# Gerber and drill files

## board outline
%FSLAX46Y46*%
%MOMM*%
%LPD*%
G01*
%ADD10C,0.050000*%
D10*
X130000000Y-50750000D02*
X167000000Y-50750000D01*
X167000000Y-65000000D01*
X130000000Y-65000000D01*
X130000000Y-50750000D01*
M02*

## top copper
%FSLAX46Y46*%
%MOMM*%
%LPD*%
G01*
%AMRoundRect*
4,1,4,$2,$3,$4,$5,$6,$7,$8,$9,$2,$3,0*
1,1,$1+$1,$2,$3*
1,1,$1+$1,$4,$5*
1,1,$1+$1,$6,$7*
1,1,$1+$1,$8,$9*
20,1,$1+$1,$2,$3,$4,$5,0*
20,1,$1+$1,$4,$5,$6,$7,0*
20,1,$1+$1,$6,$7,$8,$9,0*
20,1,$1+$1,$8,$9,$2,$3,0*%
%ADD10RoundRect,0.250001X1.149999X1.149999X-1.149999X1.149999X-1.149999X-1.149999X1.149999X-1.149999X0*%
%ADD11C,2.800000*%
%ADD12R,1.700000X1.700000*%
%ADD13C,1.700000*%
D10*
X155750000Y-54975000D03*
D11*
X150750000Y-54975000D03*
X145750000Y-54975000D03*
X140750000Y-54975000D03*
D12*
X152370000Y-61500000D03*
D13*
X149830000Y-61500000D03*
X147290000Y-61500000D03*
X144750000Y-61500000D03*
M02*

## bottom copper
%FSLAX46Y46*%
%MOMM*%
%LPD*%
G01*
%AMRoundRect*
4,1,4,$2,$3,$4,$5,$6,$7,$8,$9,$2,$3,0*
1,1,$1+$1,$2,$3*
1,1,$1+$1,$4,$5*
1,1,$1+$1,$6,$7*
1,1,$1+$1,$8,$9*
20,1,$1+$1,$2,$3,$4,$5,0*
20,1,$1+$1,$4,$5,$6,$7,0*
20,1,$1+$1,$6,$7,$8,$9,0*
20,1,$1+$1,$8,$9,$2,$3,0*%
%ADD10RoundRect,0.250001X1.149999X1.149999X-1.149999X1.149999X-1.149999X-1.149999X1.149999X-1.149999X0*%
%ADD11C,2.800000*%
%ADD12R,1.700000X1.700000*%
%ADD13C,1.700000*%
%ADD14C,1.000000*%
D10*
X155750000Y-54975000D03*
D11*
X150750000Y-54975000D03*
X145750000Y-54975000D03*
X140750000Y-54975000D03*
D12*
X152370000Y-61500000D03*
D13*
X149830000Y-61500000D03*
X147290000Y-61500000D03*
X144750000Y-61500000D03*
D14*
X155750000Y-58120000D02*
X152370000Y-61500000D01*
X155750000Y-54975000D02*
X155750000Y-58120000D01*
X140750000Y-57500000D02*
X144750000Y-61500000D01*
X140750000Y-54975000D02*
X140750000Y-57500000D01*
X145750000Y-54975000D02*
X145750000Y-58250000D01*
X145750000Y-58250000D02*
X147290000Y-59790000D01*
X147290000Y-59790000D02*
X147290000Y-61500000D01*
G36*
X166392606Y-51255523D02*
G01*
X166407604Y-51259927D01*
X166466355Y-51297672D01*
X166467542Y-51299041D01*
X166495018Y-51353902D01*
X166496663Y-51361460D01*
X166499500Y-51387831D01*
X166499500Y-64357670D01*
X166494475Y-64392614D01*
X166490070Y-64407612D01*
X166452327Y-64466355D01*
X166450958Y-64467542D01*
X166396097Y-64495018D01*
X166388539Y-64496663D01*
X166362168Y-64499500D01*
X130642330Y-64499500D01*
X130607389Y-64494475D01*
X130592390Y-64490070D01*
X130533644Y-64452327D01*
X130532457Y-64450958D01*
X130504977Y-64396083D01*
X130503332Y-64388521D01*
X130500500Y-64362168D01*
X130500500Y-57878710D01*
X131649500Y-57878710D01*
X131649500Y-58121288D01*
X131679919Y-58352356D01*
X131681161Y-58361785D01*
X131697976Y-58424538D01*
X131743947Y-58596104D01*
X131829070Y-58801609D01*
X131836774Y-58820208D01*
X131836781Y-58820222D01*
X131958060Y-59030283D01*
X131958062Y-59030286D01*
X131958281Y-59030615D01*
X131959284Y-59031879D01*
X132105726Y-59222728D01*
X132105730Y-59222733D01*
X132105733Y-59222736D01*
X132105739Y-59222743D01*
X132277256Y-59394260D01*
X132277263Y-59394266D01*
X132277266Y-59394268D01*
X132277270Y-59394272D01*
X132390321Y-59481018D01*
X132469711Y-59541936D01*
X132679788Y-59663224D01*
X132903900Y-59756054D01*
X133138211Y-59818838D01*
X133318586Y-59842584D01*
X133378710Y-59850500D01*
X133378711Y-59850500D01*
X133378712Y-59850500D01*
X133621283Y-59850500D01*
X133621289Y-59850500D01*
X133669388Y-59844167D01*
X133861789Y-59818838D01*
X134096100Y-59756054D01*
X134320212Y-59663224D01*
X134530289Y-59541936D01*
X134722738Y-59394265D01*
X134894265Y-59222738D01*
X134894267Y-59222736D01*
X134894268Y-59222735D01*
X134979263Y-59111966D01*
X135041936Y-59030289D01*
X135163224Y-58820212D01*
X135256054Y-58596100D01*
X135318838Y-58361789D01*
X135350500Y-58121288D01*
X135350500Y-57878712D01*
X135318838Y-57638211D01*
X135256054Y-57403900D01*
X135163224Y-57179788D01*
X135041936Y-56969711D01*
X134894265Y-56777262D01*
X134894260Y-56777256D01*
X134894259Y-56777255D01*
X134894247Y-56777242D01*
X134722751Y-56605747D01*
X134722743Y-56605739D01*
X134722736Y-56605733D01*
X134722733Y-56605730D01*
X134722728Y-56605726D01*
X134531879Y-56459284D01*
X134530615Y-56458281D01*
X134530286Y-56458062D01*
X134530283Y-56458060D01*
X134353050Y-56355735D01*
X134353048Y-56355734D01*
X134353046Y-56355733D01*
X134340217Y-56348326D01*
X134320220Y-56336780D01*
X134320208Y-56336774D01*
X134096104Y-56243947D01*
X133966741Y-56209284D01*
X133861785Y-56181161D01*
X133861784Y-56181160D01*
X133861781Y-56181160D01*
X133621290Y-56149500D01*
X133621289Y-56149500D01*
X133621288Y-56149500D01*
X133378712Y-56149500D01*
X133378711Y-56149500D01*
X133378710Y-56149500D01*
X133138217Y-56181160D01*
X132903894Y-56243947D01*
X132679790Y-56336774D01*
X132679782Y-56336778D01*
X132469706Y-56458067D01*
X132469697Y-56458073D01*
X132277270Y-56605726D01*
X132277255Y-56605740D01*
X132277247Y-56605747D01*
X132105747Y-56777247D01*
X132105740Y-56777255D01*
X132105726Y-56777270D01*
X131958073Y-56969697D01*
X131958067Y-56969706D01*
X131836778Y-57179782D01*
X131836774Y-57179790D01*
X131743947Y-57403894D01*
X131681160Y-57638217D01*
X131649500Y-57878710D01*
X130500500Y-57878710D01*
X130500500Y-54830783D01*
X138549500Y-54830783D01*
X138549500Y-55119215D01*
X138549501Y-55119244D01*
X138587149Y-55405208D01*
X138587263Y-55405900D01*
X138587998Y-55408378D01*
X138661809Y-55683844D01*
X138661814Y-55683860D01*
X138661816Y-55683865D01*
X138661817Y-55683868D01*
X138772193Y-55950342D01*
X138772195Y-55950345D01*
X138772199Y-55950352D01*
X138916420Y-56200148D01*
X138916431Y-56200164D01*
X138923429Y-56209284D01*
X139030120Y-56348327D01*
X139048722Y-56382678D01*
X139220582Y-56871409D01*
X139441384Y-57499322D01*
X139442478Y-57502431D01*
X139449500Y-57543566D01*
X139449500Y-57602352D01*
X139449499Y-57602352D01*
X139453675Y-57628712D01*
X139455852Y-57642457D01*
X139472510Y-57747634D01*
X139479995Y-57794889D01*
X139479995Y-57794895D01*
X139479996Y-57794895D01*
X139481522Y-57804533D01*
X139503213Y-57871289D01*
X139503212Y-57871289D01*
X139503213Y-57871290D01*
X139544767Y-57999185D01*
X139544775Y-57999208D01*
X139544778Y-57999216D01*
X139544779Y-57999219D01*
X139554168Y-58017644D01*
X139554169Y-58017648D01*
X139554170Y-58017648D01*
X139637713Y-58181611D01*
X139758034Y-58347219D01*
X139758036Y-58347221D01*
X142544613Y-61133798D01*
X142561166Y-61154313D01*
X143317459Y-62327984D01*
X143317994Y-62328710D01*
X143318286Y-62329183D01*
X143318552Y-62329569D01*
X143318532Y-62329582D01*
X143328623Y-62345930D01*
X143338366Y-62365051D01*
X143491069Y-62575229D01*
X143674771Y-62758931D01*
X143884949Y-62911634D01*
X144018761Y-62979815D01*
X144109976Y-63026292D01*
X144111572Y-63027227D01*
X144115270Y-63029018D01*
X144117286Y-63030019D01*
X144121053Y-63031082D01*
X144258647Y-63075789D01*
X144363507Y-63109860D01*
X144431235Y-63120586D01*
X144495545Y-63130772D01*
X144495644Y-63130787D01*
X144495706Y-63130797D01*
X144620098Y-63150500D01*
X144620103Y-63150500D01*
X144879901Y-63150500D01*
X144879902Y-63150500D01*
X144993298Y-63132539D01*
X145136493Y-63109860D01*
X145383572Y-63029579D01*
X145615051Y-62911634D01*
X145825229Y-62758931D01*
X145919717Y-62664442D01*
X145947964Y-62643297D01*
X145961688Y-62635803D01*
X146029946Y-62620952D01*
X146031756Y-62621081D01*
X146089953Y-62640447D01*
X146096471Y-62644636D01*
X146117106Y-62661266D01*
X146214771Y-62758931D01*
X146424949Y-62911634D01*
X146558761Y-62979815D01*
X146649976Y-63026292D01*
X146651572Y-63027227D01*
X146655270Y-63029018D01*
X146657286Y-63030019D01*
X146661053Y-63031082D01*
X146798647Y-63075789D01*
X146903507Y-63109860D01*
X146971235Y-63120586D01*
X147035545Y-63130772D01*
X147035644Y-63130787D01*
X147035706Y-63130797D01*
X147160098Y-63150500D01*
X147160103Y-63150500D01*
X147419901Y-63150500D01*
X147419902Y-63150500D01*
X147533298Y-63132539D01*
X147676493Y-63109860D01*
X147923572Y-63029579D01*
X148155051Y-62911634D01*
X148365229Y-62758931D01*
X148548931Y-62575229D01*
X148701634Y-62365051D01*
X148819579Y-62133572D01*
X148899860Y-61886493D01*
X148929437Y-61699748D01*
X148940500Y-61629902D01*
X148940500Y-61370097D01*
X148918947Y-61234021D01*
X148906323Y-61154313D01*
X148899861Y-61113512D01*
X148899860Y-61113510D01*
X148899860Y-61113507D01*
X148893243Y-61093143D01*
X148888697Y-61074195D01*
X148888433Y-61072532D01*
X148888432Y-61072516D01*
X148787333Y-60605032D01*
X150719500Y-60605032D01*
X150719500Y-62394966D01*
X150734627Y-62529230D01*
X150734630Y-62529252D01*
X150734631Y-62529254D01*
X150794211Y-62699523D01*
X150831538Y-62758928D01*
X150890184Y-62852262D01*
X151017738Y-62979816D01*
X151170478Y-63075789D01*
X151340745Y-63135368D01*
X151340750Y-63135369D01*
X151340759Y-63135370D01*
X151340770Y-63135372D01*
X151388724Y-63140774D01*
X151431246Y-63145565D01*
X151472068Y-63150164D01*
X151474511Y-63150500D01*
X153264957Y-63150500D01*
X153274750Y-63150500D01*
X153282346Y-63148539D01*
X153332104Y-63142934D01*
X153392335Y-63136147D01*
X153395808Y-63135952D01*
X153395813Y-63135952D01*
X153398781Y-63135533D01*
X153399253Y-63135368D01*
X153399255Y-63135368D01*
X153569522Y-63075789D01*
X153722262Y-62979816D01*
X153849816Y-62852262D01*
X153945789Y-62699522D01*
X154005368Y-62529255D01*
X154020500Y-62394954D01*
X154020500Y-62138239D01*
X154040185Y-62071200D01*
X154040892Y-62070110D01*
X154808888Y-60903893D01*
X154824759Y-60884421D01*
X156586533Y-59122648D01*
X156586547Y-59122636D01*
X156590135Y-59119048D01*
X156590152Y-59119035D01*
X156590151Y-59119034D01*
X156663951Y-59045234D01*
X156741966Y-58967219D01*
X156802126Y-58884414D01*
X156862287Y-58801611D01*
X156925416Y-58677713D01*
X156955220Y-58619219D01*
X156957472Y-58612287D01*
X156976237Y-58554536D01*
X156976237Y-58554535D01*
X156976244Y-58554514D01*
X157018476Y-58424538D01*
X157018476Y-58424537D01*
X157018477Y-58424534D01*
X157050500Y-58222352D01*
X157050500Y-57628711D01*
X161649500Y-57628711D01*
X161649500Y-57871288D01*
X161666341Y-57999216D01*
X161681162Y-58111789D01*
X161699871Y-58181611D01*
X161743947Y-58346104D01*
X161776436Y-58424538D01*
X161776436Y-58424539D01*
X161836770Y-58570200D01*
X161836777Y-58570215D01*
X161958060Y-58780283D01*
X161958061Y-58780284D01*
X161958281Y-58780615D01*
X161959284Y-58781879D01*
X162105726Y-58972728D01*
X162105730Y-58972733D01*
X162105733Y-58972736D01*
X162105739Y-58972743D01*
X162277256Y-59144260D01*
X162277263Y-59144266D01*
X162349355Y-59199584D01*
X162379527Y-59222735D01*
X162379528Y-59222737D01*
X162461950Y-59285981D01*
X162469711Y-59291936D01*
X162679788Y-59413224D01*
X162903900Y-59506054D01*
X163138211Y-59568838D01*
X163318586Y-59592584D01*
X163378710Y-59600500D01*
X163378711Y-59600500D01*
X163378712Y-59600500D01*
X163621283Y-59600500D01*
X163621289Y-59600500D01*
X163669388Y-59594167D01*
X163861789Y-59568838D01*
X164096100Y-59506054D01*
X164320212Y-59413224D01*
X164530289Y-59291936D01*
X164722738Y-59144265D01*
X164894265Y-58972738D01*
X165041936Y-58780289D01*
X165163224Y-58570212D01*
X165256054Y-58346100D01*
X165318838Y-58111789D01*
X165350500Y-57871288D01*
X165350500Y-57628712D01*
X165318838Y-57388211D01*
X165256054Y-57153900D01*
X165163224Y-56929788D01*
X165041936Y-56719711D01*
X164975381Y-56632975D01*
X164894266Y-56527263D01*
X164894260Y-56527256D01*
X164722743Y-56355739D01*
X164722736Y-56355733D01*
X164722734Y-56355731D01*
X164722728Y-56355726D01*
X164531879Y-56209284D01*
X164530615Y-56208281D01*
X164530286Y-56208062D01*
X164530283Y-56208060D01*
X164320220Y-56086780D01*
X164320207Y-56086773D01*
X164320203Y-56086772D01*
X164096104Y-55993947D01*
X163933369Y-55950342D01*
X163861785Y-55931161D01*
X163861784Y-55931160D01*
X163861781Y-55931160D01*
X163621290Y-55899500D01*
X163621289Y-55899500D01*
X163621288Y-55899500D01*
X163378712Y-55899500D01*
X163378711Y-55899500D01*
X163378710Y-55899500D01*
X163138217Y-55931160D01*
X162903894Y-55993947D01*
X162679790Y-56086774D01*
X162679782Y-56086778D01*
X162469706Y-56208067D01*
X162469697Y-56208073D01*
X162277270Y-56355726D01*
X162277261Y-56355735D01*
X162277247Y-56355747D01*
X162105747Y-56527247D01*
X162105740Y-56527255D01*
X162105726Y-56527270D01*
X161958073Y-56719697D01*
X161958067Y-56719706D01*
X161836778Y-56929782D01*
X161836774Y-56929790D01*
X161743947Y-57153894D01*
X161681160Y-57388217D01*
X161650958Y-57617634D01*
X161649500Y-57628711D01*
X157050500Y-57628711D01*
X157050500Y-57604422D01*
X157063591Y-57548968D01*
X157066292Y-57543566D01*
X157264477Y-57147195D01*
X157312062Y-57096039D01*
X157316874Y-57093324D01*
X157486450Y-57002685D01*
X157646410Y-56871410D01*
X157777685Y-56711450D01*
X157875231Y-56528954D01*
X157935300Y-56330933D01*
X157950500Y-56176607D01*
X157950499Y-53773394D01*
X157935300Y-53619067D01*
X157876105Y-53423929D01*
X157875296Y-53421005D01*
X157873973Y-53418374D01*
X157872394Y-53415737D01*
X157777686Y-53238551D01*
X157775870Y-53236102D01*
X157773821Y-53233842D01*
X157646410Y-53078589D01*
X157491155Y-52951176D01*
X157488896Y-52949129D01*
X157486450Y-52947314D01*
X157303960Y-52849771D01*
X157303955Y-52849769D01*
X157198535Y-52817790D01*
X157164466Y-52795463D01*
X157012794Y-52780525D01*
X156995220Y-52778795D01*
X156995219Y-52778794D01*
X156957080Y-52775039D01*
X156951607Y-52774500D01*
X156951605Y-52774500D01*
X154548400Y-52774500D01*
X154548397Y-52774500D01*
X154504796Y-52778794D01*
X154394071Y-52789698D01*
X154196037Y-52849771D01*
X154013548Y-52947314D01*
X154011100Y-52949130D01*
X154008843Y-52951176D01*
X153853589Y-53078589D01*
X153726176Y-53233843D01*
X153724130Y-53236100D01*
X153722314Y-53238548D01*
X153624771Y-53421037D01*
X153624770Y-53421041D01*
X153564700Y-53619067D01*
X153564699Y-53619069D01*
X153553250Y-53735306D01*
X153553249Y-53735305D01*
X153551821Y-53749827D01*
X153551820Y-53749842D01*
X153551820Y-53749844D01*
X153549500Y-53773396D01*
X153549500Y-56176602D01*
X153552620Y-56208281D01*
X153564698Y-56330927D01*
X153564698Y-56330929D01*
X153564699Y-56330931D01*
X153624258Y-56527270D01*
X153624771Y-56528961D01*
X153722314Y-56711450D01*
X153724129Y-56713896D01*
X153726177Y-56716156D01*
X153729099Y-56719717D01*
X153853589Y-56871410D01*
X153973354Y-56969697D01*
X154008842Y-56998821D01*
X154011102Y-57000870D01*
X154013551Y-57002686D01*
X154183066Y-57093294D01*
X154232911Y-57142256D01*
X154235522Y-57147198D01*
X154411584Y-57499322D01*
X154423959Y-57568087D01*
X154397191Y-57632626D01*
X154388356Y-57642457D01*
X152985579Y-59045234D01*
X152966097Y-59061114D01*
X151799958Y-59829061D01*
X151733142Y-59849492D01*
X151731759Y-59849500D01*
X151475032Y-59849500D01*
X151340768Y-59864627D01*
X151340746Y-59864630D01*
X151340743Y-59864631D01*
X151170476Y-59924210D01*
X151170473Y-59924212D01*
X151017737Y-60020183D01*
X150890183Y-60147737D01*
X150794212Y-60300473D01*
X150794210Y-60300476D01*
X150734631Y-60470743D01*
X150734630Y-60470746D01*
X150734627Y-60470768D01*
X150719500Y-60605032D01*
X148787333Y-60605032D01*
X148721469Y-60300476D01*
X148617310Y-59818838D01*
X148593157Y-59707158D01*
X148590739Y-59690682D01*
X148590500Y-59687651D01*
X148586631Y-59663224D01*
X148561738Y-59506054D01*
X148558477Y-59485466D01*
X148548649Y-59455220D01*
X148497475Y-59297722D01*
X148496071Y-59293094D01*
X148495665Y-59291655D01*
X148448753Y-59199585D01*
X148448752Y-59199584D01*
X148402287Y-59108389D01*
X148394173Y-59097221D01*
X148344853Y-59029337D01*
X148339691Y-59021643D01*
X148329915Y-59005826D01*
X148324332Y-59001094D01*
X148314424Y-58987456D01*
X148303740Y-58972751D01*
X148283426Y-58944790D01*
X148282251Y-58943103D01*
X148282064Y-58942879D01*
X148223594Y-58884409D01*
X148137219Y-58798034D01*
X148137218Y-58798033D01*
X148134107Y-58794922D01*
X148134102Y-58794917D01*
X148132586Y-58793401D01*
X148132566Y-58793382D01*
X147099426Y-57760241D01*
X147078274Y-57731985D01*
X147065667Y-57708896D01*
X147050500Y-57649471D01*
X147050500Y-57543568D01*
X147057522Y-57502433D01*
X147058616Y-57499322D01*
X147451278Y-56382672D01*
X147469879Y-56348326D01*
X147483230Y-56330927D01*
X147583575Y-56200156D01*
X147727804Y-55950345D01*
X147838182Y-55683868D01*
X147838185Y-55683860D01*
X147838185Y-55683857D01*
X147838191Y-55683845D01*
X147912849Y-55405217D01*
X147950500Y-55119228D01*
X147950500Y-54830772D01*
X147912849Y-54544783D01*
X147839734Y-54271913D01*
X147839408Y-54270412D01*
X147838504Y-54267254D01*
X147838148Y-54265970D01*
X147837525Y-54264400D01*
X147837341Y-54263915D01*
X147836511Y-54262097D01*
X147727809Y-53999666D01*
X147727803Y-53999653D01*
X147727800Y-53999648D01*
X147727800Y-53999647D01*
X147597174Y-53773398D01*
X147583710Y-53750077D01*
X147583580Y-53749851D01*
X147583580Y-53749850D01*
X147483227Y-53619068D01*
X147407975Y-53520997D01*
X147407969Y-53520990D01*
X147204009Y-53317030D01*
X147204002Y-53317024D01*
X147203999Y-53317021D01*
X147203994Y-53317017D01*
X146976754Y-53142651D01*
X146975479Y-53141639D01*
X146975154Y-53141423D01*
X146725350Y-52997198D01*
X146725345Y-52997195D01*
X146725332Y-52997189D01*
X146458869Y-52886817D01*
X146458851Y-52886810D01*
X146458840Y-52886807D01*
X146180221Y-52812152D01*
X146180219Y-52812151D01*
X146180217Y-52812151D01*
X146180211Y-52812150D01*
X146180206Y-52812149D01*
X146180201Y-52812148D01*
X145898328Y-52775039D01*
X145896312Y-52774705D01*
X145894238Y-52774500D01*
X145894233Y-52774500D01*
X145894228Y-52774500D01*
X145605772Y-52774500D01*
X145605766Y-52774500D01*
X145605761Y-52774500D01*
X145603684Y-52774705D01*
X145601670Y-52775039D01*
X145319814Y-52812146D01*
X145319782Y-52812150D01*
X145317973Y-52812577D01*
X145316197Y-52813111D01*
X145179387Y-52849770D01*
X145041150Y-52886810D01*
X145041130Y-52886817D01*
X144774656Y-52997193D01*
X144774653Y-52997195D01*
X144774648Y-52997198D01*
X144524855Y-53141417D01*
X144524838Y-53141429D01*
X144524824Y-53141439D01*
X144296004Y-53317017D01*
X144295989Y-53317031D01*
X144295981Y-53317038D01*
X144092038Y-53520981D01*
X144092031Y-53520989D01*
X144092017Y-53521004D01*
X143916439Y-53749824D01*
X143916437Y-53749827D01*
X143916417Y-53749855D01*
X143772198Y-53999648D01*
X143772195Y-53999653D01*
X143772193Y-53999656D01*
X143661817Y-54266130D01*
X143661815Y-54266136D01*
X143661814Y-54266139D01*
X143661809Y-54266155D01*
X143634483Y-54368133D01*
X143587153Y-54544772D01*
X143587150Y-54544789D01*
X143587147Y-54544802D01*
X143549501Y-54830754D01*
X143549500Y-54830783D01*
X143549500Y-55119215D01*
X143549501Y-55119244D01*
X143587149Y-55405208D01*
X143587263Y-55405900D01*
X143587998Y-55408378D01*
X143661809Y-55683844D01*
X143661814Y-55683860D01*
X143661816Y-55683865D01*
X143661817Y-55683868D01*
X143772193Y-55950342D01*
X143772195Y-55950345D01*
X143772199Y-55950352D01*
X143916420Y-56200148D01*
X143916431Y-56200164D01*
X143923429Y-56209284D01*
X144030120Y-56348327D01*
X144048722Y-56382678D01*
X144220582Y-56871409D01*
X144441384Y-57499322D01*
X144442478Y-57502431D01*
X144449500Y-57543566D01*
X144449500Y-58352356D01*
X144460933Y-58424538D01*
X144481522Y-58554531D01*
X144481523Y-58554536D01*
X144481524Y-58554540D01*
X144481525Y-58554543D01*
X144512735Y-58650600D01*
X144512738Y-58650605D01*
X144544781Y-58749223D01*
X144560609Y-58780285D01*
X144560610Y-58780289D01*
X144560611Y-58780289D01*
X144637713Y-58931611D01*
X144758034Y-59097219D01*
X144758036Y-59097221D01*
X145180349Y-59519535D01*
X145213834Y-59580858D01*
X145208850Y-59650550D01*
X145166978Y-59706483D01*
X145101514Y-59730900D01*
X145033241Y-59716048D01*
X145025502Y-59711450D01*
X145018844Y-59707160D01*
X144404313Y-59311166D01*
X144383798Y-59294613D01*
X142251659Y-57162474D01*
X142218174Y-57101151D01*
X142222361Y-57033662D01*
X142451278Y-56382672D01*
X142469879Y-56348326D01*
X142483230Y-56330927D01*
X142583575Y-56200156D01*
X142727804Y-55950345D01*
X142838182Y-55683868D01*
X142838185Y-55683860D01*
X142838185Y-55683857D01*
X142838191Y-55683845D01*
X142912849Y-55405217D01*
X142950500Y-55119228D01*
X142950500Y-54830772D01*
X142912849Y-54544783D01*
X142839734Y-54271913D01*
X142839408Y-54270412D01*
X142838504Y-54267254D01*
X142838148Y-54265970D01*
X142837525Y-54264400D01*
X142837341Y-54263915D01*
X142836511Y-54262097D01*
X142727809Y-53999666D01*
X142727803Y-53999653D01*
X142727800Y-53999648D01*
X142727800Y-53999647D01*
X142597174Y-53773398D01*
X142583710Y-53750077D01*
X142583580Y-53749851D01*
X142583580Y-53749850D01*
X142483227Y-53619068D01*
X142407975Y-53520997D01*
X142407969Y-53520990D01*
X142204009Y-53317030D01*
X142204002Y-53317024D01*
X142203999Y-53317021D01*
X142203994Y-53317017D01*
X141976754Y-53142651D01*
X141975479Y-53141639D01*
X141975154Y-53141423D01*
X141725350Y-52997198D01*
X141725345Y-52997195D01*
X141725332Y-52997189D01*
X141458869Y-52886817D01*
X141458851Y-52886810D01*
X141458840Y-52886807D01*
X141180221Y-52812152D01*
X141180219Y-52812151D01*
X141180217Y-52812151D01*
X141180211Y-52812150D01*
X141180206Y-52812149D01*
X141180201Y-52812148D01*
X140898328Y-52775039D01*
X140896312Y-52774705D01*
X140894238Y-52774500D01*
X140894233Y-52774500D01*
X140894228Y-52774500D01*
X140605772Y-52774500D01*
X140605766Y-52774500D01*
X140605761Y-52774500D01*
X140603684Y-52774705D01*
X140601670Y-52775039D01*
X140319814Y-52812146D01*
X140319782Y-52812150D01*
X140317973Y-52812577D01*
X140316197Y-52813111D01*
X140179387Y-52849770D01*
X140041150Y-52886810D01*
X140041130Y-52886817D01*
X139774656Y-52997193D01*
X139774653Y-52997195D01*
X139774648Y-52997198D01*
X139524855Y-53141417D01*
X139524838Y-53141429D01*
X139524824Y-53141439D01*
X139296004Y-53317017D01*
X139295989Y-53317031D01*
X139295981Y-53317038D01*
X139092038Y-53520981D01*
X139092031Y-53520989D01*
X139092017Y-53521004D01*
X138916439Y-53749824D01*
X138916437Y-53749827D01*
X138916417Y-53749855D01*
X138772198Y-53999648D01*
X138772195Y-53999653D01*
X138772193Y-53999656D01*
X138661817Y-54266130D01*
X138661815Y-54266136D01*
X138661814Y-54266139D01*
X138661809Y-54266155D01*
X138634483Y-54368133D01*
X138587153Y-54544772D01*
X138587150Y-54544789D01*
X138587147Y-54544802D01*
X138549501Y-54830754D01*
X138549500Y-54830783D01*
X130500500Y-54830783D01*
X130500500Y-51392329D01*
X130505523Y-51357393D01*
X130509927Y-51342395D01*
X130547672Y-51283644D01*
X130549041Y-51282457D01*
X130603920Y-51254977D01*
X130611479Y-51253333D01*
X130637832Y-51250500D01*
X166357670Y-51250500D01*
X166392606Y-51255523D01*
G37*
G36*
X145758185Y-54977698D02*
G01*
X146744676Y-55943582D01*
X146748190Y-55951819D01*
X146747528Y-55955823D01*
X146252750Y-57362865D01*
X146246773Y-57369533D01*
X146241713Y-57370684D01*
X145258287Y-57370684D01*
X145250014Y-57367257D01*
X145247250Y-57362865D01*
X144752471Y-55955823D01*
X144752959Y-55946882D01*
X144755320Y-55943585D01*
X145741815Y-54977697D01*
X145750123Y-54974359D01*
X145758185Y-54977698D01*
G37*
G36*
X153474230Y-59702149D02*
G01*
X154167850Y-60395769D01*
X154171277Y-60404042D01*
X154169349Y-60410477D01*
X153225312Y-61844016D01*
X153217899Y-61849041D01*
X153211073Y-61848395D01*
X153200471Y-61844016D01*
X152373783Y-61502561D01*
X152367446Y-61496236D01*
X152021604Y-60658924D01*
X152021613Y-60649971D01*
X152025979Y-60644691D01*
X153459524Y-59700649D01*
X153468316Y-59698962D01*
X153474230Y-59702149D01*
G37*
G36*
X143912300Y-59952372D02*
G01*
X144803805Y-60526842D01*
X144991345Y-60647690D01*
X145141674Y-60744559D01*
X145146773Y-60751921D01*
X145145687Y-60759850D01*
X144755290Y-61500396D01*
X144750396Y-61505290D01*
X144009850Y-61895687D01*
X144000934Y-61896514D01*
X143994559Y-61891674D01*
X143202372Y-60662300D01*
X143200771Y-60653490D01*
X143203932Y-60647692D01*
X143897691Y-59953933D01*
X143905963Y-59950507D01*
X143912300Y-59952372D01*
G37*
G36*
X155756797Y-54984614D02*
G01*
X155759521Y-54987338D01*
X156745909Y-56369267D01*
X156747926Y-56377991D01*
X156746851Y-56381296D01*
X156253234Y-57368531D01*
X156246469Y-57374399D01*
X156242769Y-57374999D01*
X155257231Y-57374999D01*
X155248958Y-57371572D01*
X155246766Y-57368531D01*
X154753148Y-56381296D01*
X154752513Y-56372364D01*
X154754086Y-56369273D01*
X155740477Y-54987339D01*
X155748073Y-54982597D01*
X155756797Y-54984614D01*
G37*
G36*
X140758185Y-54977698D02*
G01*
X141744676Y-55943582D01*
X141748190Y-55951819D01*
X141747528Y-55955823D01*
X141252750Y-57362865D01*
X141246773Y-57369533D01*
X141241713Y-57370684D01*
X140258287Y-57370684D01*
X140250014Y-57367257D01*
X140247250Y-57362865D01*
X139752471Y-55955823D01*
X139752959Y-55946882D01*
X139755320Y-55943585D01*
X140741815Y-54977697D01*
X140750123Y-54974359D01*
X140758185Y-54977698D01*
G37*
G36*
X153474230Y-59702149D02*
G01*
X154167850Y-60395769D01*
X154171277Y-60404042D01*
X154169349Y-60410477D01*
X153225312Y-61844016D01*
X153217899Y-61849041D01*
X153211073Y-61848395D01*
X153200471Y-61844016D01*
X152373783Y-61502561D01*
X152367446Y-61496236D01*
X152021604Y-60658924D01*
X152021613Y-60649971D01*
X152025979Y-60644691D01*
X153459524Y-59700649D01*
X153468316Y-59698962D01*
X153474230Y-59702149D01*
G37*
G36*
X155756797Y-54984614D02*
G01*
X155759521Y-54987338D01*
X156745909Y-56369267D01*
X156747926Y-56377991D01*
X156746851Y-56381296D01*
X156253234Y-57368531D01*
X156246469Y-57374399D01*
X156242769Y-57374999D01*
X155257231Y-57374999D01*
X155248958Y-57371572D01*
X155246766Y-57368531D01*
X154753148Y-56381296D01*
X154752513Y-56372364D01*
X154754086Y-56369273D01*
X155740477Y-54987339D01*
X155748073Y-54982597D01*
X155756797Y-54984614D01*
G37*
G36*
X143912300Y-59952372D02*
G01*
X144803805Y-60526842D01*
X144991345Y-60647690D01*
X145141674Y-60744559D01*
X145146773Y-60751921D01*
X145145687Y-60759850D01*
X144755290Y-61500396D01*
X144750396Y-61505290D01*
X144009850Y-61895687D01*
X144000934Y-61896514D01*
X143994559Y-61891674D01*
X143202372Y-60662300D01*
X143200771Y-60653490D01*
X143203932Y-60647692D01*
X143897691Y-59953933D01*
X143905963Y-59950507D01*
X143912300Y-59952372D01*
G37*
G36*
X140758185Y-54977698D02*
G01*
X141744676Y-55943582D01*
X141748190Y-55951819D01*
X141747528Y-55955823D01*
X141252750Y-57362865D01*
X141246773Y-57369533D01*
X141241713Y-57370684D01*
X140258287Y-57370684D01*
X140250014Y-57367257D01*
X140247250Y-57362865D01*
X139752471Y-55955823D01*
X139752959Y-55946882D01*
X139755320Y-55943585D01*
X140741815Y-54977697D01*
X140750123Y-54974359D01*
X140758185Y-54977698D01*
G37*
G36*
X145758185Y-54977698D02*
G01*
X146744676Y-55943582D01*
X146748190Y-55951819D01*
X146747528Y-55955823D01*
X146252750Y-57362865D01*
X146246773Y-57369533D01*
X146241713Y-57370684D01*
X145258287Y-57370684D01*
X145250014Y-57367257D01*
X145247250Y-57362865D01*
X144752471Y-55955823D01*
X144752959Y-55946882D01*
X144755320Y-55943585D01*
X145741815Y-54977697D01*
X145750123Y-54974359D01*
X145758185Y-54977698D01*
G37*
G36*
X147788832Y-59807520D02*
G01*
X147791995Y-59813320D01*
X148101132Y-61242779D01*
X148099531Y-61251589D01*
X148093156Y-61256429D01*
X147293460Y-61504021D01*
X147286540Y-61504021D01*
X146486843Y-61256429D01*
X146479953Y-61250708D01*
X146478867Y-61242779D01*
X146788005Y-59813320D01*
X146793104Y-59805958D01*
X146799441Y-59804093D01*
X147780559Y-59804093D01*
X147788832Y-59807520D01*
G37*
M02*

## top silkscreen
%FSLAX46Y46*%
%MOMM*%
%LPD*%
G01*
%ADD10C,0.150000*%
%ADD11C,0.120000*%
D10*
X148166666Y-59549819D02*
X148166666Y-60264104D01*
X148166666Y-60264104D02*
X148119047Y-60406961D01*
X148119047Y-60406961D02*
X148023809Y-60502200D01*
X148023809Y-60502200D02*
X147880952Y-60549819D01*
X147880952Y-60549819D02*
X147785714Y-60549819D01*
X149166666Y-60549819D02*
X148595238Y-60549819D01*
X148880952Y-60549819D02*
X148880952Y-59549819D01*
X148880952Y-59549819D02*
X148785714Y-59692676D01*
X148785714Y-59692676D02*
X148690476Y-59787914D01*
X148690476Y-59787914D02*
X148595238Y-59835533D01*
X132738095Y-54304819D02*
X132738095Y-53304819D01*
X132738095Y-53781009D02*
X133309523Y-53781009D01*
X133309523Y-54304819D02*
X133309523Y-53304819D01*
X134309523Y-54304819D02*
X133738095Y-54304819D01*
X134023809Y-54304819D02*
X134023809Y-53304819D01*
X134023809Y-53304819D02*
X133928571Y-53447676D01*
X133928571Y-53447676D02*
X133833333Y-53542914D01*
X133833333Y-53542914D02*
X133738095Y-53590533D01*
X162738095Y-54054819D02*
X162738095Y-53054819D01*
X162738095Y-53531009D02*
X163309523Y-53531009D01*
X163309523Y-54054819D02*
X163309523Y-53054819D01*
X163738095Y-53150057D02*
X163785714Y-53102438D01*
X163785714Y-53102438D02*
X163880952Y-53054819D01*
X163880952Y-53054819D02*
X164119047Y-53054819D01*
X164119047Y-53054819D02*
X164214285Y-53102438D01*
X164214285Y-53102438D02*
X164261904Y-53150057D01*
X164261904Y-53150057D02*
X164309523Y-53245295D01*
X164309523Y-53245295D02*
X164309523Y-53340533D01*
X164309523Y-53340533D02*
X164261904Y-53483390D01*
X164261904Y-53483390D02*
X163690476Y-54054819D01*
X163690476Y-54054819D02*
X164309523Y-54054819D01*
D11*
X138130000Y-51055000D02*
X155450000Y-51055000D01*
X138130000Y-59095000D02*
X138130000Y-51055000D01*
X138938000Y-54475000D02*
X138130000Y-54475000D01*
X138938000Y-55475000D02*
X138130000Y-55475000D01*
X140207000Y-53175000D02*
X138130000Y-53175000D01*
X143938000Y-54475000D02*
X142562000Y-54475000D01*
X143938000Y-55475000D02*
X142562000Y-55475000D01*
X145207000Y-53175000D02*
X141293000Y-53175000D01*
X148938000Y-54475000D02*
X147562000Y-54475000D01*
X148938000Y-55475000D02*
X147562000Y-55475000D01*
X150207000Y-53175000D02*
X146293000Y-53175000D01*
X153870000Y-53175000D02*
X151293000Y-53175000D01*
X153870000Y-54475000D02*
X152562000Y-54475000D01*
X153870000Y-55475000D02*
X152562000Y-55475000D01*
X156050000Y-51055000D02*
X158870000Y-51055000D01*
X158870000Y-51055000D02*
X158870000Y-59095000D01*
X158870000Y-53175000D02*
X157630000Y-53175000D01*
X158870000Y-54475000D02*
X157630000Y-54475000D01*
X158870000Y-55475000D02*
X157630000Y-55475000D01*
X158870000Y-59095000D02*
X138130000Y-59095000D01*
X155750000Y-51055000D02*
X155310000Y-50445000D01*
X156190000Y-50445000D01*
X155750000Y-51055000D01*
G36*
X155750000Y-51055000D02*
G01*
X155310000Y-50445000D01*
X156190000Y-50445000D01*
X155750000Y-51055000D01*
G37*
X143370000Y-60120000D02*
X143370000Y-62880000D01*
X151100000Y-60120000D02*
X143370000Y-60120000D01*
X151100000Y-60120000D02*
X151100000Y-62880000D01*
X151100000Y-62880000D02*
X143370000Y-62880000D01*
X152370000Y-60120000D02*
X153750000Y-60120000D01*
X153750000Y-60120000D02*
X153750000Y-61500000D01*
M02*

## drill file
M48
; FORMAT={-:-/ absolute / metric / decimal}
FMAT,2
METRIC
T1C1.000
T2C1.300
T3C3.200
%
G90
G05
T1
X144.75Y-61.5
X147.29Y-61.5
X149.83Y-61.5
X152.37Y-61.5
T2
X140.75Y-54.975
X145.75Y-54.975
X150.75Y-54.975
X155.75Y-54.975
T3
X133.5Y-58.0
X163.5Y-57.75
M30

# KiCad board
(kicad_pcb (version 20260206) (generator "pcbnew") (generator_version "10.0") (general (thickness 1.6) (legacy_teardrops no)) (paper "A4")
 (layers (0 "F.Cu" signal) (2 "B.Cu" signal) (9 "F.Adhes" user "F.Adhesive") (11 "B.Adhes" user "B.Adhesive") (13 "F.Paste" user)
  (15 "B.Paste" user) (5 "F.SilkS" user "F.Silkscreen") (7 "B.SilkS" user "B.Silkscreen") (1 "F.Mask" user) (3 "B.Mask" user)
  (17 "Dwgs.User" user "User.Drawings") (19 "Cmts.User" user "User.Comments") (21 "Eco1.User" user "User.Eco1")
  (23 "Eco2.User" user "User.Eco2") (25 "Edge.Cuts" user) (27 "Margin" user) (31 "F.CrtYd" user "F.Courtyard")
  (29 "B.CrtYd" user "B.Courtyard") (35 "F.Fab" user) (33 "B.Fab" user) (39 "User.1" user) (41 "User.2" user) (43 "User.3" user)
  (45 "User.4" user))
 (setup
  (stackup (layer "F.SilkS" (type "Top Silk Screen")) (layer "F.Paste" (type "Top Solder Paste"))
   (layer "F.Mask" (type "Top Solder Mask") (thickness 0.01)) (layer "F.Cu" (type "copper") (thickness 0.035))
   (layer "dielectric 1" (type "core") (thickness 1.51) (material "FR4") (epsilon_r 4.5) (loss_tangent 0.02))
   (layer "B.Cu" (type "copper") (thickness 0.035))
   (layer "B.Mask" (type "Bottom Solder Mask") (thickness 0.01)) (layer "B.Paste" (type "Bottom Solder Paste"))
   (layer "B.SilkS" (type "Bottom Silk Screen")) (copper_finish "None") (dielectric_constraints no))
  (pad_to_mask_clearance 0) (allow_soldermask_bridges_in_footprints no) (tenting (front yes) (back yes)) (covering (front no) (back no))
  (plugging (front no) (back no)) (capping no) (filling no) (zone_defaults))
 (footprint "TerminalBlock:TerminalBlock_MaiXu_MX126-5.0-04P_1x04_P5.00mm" (layer "F.Cu") (at 155.75 54.975 180)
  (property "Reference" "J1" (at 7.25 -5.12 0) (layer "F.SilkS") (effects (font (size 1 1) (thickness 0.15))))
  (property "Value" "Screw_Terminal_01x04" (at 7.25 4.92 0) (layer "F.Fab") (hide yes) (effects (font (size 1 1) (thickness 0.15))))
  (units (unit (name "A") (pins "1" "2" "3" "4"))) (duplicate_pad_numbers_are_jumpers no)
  (fp_line (start 17.62 3.92) (end 0.3 3.92) (stroke (width 0.12) (type solid)) (layer "F.SilkS"))
  (fp_line (start 17.62 -4.12) (end 17.62 3.92) (stroke (width 0.12) (type solid)) (layer "F.SilkS"))
  (fp_line (start 16.812 0.5) (end 17.62 0.5) (stroke (width 0.12) (type solid)) (layer "F.SilkS"))
  (fp_line (start 16.812 -0.5) (end 17.62 -0.5) (stroke (width 0.12) (type solid)) (layer "F.SilkS"))
  (fp_line (start 15.543 1.8) (end 17.62 1.8) (stroke (width 0.12) (type solid)) (layer "F.SilkS"))
  (fp_line (start 11.812 0.5) (end 13.188 0.5) (stroke (width 0.12) (type solid)) (layer "F.SilkS"))
  (fp_line (start 11.812 -0.5) (end 13.188 -0.5) (stroke (width 0.12) (type solid)) (layer "F.SilkS"))
  (fp_line (start 10.543 1.8) (end 14.457 1.8) (stroke (width 0.12) (type solid)) (layer "F.SilkS"))
  (fp_line (start 6.812 0.5) (end 8.188 0.5) (stroke (width 0.12) (type solid)) (layer "F.SilkS"))
  (fp_line (start 6.812 -0.5) (end 8.188 -0.5) (stroke (width 0.12) (type solid)) (layer "F.SilkS"))
  (fp_line (start 5.543 1.8) (end 9.457 1.8) (stroke (width 0.12) (type solid)) (layer "F.SilkS"))
  (fp_line (start 1.88 1.8) (end 4.457 1.8) (stroke (width 0.12) (type solid)) (layer "F.SilkS"))
  (fp_line (start 1.88 0.5) (end 3.188 0.5) (stroke (width 0.12) (type solid)) (layer "F.SilkS"))
  (fp_line (start 1.88 -0.5) (end 3.188 -0.5) (stroke (width 0.12) (type solid)) (layer "F.SilkS"))
  (fp_line (start -0.3 3.92) (end -3.12 3.92) (stroke (width 0.12) (type solid)) (layer "F.SilkS"))
  (fp_line (start -3.12 3.92) (end -3.12 -4.12) (stroke (width 0.12) (type solid)) (layer "F.SilkS"))
  (fp_line (start -3.12 1.8) (end -1.88 1.8) (stroke (width 0.12) (type solid)) (layer "F.SilkS"))
  (fp_line (start -3.12 0.5) (end -1.88 0.5) (stroke (width 0.12) (type solid)) (layer "F.SilkS"))
  (fp_line (start -3.12 -0.5) (end -1.88 -0.5) (stroke (width 0.12) (type solid)) (layer "F.SilkS"))
  (fp_line (start -3.12 -4.12) (end 17.62 -4.12) (stroke (width 0.12) (type solid)) (layer "F.SilkS"))
  (fp_poly (pts (xy 0 3.92) (xy 0.44 4.53) (xy -0.44 4.53)) (stroke (width 0.12) (type solid)) (fill yes) (layer "F.SilkS"))
  (pad "1" thru_hole roundrect (at 0 0 180) (size 2.8 2.8) (drill 1.3) (layers "*.Cu" "*.Mask") (remove_unused_layers no)
   (roundrect_rratio 0.089286) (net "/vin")
   (teardrops (best_length_ratio 0.5) (max_length 1) (best_width_ratio 1) (max_width 2) (curved_edges no) (filter_ratio 0.9) (enabled yes)
    (allow_two_segments yes) (prefer_zone_connections yes)))
  (pad "2" thru_hole circle (at 5 0 180) (size 2.8 2.8) (drill 1.3) (layers "*.Cu" "*.Mask") (remove_unused_layers no) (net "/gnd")
   (teardrops (best_length_ratio 0.5) (max_length 1) (best_width_ratio 1) (max_width 2) (curved_edges no) (filter_ratio 0.9) (enabled yes)
    (allow_two_segments yes) (prefer_zone_connections yes)))
  (pad "3" thru_hole circle (at 10 0 180) (size 2.8 2.8) (drill 1.3) (layers "*.Cu" "*.Mask") (remove_unused_layers no) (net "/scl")
   (teardrops (best_length_ratio 0.5) (max_length 1) (best_width_ratio 1) (max_width 2) (curved_edges no) (filter_ratio 0.9) (enabled yes)
    (allow_two_segments yes) (prefer_zone_connections yes)))
  (pad "4" thru_hole circle (at 15 0 180) (size 2.8 2.8) (drill 1.3) (layers "*.Cu" "*.Mask") (remove_unused_layers no) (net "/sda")
   (teardrops (best_length_ratio 0.5) (max_length 1) (best_width_ratio 1) (max_width 2) (curved_edges no) (filter_ratio 0.9) (enabled yes)
    (allow_two_segments yes) (prefer_zone_connections yes))))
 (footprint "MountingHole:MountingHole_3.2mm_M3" (layer "F.Cu") (at 133.5 58)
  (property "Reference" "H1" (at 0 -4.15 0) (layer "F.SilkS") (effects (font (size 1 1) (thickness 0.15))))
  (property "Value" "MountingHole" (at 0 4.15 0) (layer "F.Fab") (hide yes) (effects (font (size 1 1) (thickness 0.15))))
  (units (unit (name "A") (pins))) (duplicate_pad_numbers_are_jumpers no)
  (pad "" np_thru_hole circle (at 0 0) (size 3.2 3.2) (drill 3.2) (layers "*.Cu" "*.Mask")))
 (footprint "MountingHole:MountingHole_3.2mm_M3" (layer "F.Cu") (at 163.5 57.75)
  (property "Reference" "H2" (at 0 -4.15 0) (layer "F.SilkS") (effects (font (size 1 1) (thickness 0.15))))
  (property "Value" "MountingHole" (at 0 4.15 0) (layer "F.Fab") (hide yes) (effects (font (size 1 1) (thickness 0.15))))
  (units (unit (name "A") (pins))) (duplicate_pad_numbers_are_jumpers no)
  (pad "" np_thru_hole circle (at 0 0) (size 3.2 3.2) (drill 3.2) (layers "*.Cu" "*.Mask")))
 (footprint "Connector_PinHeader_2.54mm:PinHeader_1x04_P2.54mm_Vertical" (layer "F.Cu") (at 152.37 61.5 -90)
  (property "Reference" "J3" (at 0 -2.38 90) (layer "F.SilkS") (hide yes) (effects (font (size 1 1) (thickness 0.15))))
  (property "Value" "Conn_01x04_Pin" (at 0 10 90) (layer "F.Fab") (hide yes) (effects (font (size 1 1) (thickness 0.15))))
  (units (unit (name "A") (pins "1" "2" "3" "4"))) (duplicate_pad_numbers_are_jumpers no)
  (fp_line (start -1.38 9) (end 1.38 9) (stroke (width 0.12) (type solid)) (layer "F.SilkS"))
  (fp_line (start -1.38 1.27) (end -1.38 9) (stroke (width 0.12) (type solid)) (layer "F.SilkS"))
  (fp_line (start -1.38 1.27) (end 1.38 1.27) (stroke (width 0.12) (type solid)) (layer "F.SilkS"))
  (fp_line (start 1.38 1.27) (end 1.38 9) (stroke (width 0.12) (type solid)) (layer "F.SilkS"))
  (fp_line (start -1.38 0) (end -1.38 -1.38) (stroke (width 0.12) (type solid)) (layer "F.SilkS"))
  (fp_line (start -1.38 -1.38) (end 0 -1.38) (stroke (width 0.12) (type solid)) (layer "F.SilkS"))
  (pad "1" thru_hole rect (at 0 0 270) (size 1.7 1.7) (drill 1) (layers "*.Cu" "*.Mask") (remove_unused_layers no) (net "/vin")
   (teardrops (best_length_ratio 0.5) (max_length 1) (best_width_ratio 1) (max_width 2) (curved_edges no) (filter_ratio 0.9) (enabled yes)
    (allow_two_segments yes) (prefer_zone_connections yes)))
  (pad "2" thru_hole circle (at 0 2.54 270) (size 1.7 1.7) (drill 1) (layers "*.Cu" "*.Mask") (remove_unused_layers no) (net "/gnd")
   (teardrops (best_length_ratio 0.5) (max_length 1) (best_width_ratio 1) (max_width 2) (curved_edges no) (filter_ratio 0.9) (enabled yes)
    (allow_two_segments yes) (prefer_zone_connections yes)))
  (pad "3" thru_hole circle (at 0 5.08 270) (size 1.7 1.7) (drill 1) (layers "*.Cu" "*.Mask") (remove_unused_layers no) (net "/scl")
   (teardrops (best_length_ratio 0.5) (max_length 1) (best_width_ratio 1) (max_width 2) (curved_edges no) (filter_ratio 0.9) (enabled yes)
    (allow_two_segments yes) (prefer_zone_connections yes)))
  (pad "4" thru_hole circle (at 0 7.62 270) (size 1.7 1.7) (drill 1) (layers "*.Cu" "*.Mask") (remove_unused_layers no) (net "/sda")
   (teardrops (best_length_ratio 0.5) (max_length 1) (best_width_ratio 1) (max_width 2) (curved_edges no) (filter_ratio 0.9) (enabled yes)
    (allow_two_segments yes) (prefer_zone_connections yes))))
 (gr_rect (start 130 50.75) (end 167 65) (stroke (width 0.05) (type default)) (fill no) (layer "Edge.Cuts"))
 (segment (start 155.75 58.12) (end 152.37 61.5) (width 1) (layer "B.Cu") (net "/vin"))
 (segment (start 155.75 54.975) (end 155.75 58.12) (width 1) (layer "B.Cu") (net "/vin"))
 (segment (start 140.75 57.5) (end 144.75 61.5) (width 1) (layer "B.Cu") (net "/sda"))
 (segment (start 140.75 54.975) (end 140.75 57.5) (width 1) (layer "B.Cu") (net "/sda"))
 (segment (start 145.75 54.975) (end 145.75 58.25) (width 1) (layer "B.Cu") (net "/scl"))
 (segment (start 145.75 58.25) (end 147.29 59.79) (width 1) (layer "B.Cu") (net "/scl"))
 (segment (start 147.29 59.79) (end 147.29 61.5) (width 1) (layer "B.Cu") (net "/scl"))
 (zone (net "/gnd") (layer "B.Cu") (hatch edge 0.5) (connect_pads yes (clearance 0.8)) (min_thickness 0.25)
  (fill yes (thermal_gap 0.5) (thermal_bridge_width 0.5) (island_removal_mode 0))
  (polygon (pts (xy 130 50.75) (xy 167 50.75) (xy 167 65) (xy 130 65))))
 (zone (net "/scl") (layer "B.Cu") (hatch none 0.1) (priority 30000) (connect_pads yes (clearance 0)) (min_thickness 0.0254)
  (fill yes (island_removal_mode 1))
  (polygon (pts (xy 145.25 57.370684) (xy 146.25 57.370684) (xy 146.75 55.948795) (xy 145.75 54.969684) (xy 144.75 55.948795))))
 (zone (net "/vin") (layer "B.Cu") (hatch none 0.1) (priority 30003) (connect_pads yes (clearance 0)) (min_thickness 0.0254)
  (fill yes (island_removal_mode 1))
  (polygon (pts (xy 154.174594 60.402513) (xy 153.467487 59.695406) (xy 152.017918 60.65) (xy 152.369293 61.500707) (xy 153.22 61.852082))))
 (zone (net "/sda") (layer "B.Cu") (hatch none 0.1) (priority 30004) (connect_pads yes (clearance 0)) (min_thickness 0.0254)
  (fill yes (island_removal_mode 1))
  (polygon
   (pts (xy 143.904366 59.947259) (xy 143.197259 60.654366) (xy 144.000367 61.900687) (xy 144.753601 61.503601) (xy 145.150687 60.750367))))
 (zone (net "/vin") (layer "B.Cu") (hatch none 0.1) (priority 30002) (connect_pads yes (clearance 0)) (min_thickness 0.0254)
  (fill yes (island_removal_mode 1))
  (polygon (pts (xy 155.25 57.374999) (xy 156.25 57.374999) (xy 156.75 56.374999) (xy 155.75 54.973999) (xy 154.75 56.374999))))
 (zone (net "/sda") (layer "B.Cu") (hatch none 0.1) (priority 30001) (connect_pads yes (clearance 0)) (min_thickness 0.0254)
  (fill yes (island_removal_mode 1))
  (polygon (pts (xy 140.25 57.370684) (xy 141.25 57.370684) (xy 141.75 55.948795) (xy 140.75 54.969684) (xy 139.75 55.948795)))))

